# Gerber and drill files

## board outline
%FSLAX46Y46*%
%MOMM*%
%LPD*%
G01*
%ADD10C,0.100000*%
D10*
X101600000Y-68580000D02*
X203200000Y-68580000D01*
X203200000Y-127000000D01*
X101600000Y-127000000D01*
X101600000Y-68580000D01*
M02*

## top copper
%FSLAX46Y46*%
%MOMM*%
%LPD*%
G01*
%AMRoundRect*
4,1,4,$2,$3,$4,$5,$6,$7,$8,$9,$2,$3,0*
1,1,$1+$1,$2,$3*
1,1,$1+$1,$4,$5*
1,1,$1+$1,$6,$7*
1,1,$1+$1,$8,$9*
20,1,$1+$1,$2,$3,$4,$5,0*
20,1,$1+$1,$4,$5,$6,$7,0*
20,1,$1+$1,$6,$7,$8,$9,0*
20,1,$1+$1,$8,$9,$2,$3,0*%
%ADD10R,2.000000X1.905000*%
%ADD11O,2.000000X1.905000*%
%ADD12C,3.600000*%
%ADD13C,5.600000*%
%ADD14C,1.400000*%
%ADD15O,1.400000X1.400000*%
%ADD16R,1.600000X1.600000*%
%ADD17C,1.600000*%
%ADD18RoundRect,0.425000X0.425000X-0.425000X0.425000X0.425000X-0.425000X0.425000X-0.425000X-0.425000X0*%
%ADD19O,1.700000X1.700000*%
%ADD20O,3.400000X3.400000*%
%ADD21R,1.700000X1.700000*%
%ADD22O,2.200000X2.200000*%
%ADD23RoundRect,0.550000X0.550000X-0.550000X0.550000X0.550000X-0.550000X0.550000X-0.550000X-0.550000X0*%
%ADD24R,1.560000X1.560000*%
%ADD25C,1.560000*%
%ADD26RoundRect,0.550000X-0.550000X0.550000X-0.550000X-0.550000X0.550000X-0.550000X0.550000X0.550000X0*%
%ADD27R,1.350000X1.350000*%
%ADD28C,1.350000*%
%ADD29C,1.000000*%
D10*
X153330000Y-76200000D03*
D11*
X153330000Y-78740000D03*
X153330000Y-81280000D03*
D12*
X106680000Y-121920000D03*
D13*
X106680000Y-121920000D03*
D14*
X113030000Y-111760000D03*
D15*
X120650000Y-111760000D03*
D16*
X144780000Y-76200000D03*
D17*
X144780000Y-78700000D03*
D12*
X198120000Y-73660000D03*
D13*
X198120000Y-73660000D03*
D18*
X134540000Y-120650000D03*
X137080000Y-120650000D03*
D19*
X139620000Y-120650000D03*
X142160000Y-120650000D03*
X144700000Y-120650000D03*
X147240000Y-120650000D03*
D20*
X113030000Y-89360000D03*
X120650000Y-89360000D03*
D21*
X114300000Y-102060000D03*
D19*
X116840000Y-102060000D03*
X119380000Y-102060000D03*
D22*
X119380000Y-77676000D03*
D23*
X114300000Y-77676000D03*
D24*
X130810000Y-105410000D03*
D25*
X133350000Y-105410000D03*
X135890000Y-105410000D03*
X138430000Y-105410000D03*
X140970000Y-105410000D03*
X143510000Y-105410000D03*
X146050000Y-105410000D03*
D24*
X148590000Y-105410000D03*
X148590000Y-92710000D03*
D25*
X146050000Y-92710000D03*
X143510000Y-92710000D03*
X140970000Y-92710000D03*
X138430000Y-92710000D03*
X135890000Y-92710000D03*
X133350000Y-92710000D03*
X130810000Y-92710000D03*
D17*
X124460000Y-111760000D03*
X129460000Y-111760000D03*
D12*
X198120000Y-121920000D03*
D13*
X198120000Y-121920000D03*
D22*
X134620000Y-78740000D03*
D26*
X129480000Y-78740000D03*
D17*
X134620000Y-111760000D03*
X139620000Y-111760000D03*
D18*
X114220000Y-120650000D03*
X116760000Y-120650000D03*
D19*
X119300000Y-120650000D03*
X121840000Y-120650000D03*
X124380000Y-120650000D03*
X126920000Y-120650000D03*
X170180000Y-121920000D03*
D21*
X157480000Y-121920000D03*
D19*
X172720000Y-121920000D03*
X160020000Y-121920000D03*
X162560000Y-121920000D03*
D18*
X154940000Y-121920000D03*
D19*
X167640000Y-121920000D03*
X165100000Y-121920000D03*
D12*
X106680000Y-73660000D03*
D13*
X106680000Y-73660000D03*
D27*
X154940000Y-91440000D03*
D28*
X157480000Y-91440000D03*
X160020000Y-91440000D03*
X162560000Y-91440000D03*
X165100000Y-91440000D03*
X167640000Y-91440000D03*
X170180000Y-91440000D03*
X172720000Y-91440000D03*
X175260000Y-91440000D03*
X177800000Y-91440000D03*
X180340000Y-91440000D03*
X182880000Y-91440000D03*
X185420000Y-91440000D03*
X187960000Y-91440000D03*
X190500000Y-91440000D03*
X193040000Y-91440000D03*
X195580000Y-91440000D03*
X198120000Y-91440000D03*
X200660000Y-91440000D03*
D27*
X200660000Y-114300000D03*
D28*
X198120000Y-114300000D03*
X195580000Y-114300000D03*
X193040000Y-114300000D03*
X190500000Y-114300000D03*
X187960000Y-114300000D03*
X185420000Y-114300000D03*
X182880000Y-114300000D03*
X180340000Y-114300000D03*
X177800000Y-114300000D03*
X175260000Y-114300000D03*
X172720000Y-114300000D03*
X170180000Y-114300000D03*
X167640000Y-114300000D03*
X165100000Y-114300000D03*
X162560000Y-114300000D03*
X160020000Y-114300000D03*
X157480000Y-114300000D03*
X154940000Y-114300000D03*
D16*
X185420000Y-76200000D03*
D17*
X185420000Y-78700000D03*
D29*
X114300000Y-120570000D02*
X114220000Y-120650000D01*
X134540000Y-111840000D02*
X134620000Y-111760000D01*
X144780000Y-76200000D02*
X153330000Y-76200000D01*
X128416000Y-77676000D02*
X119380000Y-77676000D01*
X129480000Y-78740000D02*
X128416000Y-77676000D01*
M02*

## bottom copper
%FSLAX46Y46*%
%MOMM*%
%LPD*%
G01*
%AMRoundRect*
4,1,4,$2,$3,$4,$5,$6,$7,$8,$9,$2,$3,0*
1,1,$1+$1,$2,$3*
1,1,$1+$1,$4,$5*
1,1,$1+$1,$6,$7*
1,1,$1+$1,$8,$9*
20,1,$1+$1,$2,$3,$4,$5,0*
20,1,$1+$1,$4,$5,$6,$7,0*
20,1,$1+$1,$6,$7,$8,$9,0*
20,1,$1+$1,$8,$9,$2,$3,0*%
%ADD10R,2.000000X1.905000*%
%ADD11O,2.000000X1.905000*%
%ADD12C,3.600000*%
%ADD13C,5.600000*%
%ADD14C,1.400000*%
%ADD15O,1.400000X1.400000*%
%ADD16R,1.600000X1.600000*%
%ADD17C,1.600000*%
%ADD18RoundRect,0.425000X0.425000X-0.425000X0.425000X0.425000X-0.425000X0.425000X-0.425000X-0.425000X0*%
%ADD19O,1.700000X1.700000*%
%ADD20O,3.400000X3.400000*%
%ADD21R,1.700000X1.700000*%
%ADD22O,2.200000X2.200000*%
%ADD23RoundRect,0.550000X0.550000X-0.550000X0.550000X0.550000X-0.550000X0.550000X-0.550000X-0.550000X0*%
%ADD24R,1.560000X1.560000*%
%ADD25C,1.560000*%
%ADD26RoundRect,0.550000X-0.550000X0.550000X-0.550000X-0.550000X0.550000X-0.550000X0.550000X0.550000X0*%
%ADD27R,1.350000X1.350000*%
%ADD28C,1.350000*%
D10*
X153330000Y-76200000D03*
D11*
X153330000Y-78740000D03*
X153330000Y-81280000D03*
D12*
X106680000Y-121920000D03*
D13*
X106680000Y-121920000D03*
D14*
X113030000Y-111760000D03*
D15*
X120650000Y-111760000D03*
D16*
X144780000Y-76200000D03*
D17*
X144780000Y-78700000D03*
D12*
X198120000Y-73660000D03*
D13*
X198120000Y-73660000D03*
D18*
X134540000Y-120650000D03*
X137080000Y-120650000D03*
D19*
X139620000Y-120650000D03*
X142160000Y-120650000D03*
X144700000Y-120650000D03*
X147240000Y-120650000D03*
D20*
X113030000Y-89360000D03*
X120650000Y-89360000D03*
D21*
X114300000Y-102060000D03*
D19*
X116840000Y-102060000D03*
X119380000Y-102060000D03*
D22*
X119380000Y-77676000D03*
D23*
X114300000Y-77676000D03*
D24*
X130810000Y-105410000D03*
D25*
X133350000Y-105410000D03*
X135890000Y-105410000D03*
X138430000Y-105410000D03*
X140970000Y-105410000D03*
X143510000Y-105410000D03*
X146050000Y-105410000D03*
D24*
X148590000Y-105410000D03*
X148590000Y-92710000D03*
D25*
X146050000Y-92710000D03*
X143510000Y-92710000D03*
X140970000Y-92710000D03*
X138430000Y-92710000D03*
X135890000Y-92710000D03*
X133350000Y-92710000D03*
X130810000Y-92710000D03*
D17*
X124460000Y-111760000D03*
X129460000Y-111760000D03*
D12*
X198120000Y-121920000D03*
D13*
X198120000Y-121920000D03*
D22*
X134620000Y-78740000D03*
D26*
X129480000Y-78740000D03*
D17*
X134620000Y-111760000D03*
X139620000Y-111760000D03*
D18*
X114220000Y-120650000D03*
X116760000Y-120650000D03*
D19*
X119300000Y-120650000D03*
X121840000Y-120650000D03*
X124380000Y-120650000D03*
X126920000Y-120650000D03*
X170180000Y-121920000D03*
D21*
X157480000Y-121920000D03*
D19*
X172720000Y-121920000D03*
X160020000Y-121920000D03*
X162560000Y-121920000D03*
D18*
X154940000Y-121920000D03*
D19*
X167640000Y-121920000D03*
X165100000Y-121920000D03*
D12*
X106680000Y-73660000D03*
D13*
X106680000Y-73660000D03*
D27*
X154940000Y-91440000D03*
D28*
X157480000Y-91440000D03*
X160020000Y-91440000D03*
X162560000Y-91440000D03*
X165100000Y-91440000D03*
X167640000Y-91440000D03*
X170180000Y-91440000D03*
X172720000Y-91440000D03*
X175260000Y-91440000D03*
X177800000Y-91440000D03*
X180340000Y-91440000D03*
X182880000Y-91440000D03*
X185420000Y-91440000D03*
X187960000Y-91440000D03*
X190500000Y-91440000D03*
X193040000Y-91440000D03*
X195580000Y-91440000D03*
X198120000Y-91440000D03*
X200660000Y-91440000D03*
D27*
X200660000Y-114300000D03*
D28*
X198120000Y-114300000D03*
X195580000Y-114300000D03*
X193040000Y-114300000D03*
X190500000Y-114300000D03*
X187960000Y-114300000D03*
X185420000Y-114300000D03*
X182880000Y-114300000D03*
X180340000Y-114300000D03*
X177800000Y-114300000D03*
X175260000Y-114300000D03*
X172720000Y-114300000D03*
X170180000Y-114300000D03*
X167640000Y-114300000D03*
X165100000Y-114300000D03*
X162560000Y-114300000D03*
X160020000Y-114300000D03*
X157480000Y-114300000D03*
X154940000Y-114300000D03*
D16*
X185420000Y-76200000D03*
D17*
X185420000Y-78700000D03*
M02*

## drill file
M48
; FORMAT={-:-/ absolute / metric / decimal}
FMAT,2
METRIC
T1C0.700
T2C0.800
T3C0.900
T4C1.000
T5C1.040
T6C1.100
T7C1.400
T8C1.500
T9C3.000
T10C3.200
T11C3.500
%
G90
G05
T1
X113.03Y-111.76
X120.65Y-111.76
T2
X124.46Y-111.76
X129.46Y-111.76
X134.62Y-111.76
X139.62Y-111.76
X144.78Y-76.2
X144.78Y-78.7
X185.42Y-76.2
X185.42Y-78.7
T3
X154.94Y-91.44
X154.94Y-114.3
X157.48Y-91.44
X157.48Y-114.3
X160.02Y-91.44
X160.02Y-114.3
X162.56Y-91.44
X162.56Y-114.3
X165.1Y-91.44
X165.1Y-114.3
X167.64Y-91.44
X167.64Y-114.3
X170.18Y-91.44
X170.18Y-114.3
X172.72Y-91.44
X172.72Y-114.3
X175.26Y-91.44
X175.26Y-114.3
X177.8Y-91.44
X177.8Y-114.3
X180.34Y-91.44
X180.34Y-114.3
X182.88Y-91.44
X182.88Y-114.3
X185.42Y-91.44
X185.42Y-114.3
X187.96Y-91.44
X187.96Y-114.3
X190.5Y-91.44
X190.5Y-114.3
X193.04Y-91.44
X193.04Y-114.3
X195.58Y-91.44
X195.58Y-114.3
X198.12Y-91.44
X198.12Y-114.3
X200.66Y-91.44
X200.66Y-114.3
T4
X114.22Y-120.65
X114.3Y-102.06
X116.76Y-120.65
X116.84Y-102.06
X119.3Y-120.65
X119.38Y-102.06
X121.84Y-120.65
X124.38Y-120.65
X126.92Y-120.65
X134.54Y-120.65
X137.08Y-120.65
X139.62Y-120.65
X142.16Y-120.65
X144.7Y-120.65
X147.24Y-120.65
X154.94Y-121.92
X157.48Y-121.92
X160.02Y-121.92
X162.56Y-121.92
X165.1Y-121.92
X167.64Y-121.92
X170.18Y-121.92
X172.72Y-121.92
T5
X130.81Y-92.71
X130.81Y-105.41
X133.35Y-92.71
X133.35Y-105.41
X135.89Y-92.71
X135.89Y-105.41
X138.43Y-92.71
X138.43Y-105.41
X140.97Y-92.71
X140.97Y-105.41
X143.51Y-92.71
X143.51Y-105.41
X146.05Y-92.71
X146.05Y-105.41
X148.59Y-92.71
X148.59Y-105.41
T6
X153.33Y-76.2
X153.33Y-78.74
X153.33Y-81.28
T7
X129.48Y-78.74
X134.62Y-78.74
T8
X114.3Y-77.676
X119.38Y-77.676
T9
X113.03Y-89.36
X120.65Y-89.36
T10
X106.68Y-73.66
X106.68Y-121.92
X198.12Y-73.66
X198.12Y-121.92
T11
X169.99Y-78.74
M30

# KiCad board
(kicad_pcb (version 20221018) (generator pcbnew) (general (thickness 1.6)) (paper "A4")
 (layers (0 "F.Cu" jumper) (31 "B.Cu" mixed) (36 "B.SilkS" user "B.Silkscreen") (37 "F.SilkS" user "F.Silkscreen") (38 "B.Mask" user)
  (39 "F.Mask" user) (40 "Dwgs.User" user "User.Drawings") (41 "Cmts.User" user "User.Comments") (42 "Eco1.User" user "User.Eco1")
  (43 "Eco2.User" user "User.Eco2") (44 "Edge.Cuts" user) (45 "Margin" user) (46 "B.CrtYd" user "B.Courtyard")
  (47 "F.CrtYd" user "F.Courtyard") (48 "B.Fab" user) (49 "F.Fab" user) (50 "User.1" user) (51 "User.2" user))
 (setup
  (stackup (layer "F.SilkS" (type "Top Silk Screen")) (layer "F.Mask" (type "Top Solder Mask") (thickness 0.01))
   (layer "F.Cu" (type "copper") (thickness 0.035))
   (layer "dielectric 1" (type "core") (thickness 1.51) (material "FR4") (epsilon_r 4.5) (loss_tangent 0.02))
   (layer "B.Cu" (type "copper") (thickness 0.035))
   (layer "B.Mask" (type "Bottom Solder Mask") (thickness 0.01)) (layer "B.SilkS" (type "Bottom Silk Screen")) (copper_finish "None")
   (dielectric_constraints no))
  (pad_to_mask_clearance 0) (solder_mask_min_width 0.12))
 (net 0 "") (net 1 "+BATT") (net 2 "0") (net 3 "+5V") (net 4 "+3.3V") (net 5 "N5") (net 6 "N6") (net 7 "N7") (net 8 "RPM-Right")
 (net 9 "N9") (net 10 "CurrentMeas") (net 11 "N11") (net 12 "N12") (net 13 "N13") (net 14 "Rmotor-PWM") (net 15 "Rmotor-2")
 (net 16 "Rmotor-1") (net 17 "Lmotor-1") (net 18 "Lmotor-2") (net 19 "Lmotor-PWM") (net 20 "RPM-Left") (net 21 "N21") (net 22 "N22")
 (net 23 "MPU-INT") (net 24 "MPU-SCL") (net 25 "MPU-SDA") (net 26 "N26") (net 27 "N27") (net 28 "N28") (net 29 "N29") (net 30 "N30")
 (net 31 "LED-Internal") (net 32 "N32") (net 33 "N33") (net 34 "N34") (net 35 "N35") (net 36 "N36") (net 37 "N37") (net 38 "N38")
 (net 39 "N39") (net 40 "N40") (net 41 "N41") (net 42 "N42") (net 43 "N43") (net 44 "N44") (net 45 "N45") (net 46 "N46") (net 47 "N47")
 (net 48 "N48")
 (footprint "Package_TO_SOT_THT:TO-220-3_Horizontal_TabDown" (layer "F.Cu") (at 153.33 76.2 -90)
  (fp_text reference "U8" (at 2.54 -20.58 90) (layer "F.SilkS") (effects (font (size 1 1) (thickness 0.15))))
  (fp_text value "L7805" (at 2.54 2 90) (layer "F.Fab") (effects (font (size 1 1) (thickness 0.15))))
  (pad "" np_thru_hole oval (at 2.54 -16.66 270) (size 3.5 3.5) (drill 3.5) (layers "*.Cu" "*.Mask"))
  (pad "1" thru_hole rect (at 0 0 270) (size 1.905 2) (drill 1.1) (layers "*.Cu" "*.Mask") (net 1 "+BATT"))
  (pad "2" thru_hole oval (at 2.54 0 270) (size 1.905 2) (drill 1.1) (layers "*.Cu" "*.Mask") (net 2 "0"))
  (pad "3" thru_hole oval (at 5.08 0 270) (size 1.905 2) (drill 1.1) (layers "*.Cu" "*.Mask") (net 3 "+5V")))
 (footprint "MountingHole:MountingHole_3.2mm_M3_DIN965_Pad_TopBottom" (layer "F.Cu") (at 106.68 121.92)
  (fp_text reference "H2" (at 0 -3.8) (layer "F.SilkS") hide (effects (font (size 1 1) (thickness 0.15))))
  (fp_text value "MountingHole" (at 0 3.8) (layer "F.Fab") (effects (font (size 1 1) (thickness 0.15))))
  (pad "1" thru_hole circle (at 0 0) (size 3.6 3.6) (drill 3.2) (layers "*.Cu" "*.Mask"))
  (pad "1" connect circle (at 0 0) (size 5.6 5.6) (layers "F.Cu" "F.Mask"))
  (pad "1" connect circle (at 0 0) (size 5.6 5.6) (layers "B.Cu" "B.Mask")))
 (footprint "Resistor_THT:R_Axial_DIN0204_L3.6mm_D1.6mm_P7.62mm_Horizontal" (layer "F.Cu") (at 113.03 111.76)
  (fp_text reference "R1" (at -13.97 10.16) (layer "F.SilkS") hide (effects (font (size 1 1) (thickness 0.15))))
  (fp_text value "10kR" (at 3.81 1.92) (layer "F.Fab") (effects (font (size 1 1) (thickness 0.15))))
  (pad "1" thru_hole circle (at 0 0) (size 1.4 1.4) (drill 0.7) (layers "*.Cu" "*.Mask") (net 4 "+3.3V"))
  (pad "2" thru_hole oval (at 7.62 0) (size 1.4 1.4) (drill 0.7) (layers "*.Cu" "*.Mask") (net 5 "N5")))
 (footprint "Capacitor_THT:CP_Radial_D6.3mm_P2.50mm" (layer "F.Cu") (at 144.78 76.2 -90)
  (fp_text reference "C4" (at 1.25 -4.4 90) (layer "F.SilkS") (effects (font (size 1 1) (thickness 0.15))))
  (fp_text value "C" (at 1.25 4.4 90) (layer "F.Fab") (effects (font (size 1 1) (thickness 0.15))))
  (pad "1" thru_hole rect (at 0 0 270) (size 1.6 1.6) (drill 0.8) (layers "*.Cu" "*.Mask") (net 1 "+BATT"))
  (pad "2" thru_hole circle (at 2.5 0 270) (size 1.6 1.6) (drill 0.8) (layers "*.Cu" "*.Mask") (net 2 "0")))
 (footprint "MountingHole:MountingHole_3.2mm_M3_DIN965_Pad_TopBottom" (layer "F.Cu") (at 198.12 73.66)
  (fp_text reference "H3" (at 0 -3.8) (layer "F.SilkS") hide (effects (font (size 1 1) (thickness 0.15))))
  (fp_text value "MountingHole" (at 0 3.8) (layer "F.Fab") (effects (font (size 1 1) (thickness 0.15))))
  (pad "1" thru_hole circle (at 0 0) (size 3.6 3.6) (drill 3.2) (layers "*.Cu" "*.Mask"))
  (pad "1" connect circle (at 0 0) (size 5.6 5.6) (layers "F.Cu" "F.Mask"))
  (pad "1" connect circle (at 0 0) (size 5.6 5.6) (layers "B.Cu" "B.Mask")))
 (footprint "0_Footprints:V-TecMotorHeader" (layer "F.Cu") (at 141.2075 119.38 90)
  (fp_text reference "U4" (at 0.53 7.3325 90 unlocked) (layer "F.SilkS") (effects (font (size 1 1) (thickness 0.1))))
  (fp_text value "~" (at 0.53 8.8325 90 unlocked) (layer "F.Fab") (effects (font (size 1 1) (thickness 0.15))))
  (pad "1" thru_hole roundrect (at -1.27 -6.6675 90) (size 1.7 1.7) (drill 1) (layers "*.Cu" "*.Mask") (roundrect_rratio 0.25) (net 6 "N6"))
  (pad "2" thru_hole roundrect (at -1.27 -4.1275 90) (size 1.7 1.7) (drill 1) (layers "*.Cu" "*.Mask") (roundrect_rratio 0.25) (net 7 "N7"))
  (pad "3" thru_hole oval (at -1.27 -1.5875 90) (size 1.7 1.7) (drill 1) (layers "*.Cu" "*.Mask") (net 4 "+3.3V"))
  (pad "4" thru_hole oval (at -1.27 0.9525 90) (size 1.7 1.7) (drill 1) (layers "*.Cu" "*.Mask") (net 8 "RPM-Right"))
  (pad "5" thru_hole oval (at -1.27 3.4925 90) (size 1.7 1.7) (drill 1) (layers "*.Cu" "*.Mask") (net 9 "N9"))
  (pad "6" thru_hole oval (at -1.27 6.0325 90) (size 1.7 1.7) (drill 1) (layers "*.Cu" "*.Mask") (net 2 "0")))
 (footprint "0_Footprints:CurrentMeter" (layer "F.Cu") (at 116.84 102.06)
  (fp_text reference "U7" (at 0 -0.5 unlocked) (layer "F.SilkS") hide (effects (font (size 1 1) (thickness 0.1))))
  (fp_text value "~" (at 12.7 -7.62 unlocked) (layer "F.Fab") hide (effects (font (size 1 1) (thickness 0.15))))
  (pad "" thru_hole oval (at -3.81 -12.7 90) (size 3.4 3.4) (drill 3) (layers "*.Cu" "*.Mask"))
  (pad "" thru_hole oval (at 3.81 -12.7 90) (size 3.4 3.4) (drill 3) (layers "*.Cu" "*.Mask"))
  (pad "1" thru_hole rect (at -2.54 0 90) (size 1.7 1.7) (drill 1) (layers "*.Cu" "*.Mask") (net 2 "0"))
  (pad "2" thru_hole oval (at 0 0 90) (size 1.7 1.7) (drill 1) (layers "*.Cu" "*.Mask") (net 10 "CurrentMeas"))
  (pad "3" thru_hole oval (at 2.54 0 90) (size 1.7 1.7) (drill 1) (layers "*.Cu" "*.Mask") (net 3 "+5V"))
  (pad "p1" thru_hole oval (at 2.54 -24.384 90) (size 2.2 2.2) (drill 1.5) (layers "*.Cu" "*.Mask") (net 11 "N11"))
  (pad "p2" thru_hole roundrect (at -2.54 -24.384 90) (size 2.2 2.2) (drill 1.5) (layers "*.Cu" "*.Mask") (roundrect_rratio 0.25)
   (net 1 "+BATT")))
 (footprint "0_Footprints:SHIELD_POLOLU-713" (layer "F.Cu") (at 139.7 99.06 90)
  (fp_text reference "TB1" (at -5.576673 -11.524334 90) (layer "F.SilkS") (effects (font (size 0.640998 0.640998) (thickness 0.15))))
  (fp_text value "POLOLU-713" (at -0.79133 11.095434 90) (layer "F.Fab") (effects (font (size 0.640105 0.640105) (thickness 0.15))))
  (pad "1" thru_hole rect (at -6.35 -8.89 90) (size 1.56 1.56) (drill 1.04) (layers "*.Cu" "*.Mask") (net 2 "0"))
  (pad "2" thru_hole circle (at -6.35 -6.35 90) (size 1.56 1.56) (drill 1.04) (layers "*.Cu" "*.Mask") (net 4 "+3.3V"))
  (pad "3" thru_hole circle (at -6.35 -3.81 90) (size 1.56 1.56) (drill 1.04) (layers "*.Cu" "*.Mask") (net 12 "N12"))
  (pad "4" thru_hole circle (at -6.35 -1.27 90) (size 1.56 1.56) (drill 1.04) (layers "*.Cu" "*.Mask") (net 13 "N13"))
  (pad "5" thru_hole circle (at -6.35 1.27 90) (size 1.56 1.56) (drill 1.04) (layers "*.Cu" "*.Mask") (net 6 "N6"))
  (pad "6" thru_hole circle (at -6.35 3.81 90) (size 1.56 1.56) (drill 1.04) (layers "*.Cu" "*.Mask") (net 7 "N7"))
  (pad "7" thru_hole circle (at -6.35 6.35 90) (size 1.56 1.56) (drill 1.04) (layers "*.Cu" "*.Mask") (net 1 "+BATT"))
  (pad "8" thru_hole rect (at -6.35 8.89 90) (size 1.56 1.56) (drill 1.04) (layers "*.Cu" "*.Mask") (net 2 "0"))
  (pad "9" thru_hole rect (at 6.35 8.89 90) (size 1.56 1.56) (drill 1.04) (layers "*.Cu" "*.Mask") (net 2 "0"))
  (pad "10" thru_hole circle (at 6.35 6.35 90) (size 1.56 1.56) (drill 1.04) (layers "*.Cu" "*.Mask") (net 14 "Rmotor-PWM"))
  (pad "11" thru_hole circle (at 6.35 3.81 90) (size 1.56 1.56) (drill 1.04) (layers "*.Cu" "*.Mask") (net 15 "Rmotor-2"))
  (pad "12" thru_hole circle (at 6.35 1.27 90) (size 1.56 1.56) (drill 1.04) (layers "*.Cu" "*.Mask") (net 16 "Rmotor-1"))
  (pad "13" thru_hole circle (at 6.35 -1.27 90) (size 1.56 1.56) (drill 1.04) (layers "*.Cu" "*.Mask") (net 5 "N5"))
  (pad "14" thru_hole circle (at 6.35 -3.81 90) (size 1.56 1.56) (drill 1.04) (layers "*.Cu" "*.Mask") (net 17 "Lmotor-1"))
  (pad "15" thru_hole circle (at 6.35 -6.35 90) (size 1.56 1.56) (drill 1.04) (layers "*.Cu" "*.Mask") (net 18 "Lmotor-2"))
  (pad "16" thru_hole circle (at 6.35 -8.89 90) (size 1.56 1.56) (drill 1.04) (layers "*.Cu" "*.Mask") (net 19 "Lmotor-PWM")))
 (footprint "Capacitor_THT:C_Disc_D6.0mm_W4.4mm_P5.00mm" (layer "F.Cu") (at 124.46 111.76)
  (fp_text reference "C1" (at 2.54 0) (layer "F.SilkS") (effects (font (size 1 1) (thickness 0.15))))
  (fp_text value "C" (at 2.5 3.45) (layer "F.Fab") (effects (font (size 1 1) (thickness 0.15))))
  (pad "1" thru_hole circle (at 0 0) (size 1.6 1.6) (drill 0.8) (layers "*.Cu" "*.Mask") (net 12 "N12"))
  (pad "2" thru_hole circle (at 5 0) (size 1.6 1.6) (drill 0.8) (layers "*.Cu" "*.Mask") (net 13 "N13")))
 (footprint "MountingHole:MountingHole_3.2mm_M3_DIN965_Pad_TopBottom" (layer "F.Cu") (at 198.12 121.92)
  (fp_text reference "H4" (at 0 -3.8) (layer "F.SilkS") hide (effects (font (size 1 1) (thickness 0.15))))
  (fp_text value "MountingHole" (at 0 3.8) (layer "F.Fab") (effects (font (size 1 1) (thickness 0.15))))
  (pad "1" thru_hole circle (at 0 0) (size 3.6 3.6) (drill 3.2) (layers "*.Cu" "*.Mask"))
  (pad "1" connect circle (at 0 0) (size 5.6 5.6) (layers "F.Cu" "F.Mask"))
  (pad "1" connect circle (at 0 0) (size 5.6 5.6) (layers "B.Cu" "B.Mask")))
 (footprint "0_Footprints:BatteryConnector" (layer "F.Cu") (at 130.115 78.74 -90)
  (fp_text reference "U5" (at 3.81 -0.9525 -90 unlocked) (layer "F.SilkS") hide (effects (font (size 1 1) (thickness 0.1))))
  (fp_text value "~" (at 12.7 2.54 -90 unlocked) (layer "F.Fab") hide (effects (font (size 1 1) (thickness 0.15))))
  (pad "GND" thru_hole oval (at 0 -4.505 270) (size 2.2 2.2) (drill 1.4) (layers "*.Cu" "*.Mask") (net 2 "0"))
  (pad "Vbatt" thru_hole roundrect (at 0 0.635 270) (size 2.2 2.2) (drill 1.4) (layers "*.Cu" "*.Mask") (roundrect_rratio 0.25)
   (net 11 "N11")))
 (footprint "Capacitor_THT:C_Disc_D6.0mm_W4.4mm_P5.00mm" (layer "F.Cu") (at 134.62 111.76)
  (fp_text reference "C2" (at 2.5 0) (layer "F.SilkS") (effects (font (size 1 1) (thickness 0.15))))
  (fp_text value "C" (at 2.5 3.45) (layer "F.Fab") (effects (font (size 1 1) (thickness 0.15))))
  (pad "1" thru_hole circle (at 0 0) (size 1.6 1.6) (drill 0.8) (layers "*.Cu" "*.Mask") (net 6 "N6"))
  (pad "2" thru_hole circle (at 5 0) (size 1.6 1.6) (drill 0.8) (layers "*.Cu" "*.Mask") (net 7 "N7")))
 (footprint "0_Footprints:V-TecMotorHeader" (layer "F.Cu") (at 120.8875 119.38 90)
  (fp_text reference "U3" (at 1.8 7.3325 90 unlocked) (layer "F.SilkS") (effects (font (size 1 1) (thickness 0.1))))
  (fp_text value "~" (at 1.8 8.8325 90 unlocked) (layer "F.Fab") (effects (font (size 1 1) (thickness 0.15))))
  (pad "1" thru_hole roundrect (at -1.27 -6.6675 90) (size 1.7 1.7) (drill 1) (layers "*.Cu" "*.Mask") (roundrect_rratio 0.25)
   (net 12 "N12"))
  (pad "2" thru_hole roundrect (at -1.27 -4.1275 90) (size 1.7 1.7) (drill 1) (layers "*.Cu" "*.Mask") (roundrect_rratio 0.25)
   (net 13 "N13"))
  (pad "3" thru_hole oval (at -1.27 -1.5875 90) (size 1.7 1.7) (drill 1) (layers "*.Cu" "*.Mask") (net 4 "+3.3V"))
  (pad "4" thru_hole oval (at -1.27 0.9525 90) (size 1.7 1.7) (drill 1) (layers "*.Cu" "*.Mask") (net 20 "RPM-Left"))
  (pad "5" thru_hole oval (at -1.27 3.4925 90) (size 1.7 1.7) (drill 1) (layers "*.Cu" "*.Mask") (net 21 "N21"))
  (pad "6" thru_hole oval (at -1.27 6.0325 90) (size 1.7 1.7) (drill 1) (layers "*.Cu" "*.Mask") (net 2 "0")))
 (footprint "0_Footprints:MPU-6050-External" (layer "F.Cu") (at 172.72 121.92 -90)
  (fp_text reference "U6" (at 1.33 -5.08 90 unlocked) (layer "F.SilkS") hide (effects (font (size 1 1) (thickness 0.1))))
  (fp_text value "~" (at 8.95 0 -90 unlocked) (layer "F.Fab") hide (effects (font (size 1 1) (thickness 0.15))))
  (pad "ADO" thru_hole oval (at 0 2.54 90) (size 1.7 1.7) (drill 1) (layers "*.Cu" "*.Mask") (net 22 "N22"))
  (pad "GND" thru_hole rect (at 0 15.24 90) (size 1.7 1.7) (drill 1) (layers "*.Cu" "*.Mask") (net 2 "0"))
  (pad "INT" thru_hole oval (at 0 0 90) (size 1.7 1.7) (drill 1) (layers "*.Cu" "*.Mask") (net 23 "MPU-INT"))
  (pad "SCL" thru_hole oval (at 0 12.7 90) (size 1.7 1.7) (drill 1) (layers "*.Cu" "*.Mask") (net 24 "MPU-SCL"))
  (pad "SDA" thru_hole oval (at 0 10.16 90) (size 1.7 1.7) (drill 1) (layers "*.Cu" "*.Mask") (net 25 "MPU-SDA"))
  (pad "VCC" thru_hole roundrect (at 0 17.78 90) (size 1.7 1.7) (drill 1) (layers "*.Cu" "*.Mask") (roundrect_rratio 0.25) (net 4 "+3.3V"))
  (pad "XCL" thru_hole oval (at 0 5.08 90) (size 1.7 1.7) (drill 1) (layers "*.Cu" "*.Mask") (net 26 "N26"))
  (pad "XDA" thru_hole oval (at 0 7.62 90) (size 1.7 1.7) (drill 1) (layers "*.Cu" "*.Mask") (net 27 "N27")))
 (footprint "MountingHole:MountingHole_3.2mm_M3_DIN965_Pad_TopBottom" (layer "F.Cu") (at 106.68 73.66)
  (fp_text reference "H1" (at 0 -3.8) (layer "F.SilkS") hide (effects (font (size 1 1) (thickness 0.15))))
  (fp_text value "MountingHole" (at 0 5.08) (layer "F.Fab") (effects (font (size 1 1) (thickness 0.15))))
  (pad "1" thru_hole circle (at 0 0) (size 3.6 3.6) (drill 3.2) (layers "*.Cu" "*.Mask"))
  (pad "1" connect circle (at 0 0) (size 5.6 5.6) (layers "F.Cu" "F.Mask"))
  (pad "1" connect circle (at 0 0) (size 5.6 5.6) (layers "B.Cu" "B.Mask")))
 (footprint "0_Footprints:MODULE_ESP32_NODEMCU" (layer "F.Cu") (at 177.8 102.87 90)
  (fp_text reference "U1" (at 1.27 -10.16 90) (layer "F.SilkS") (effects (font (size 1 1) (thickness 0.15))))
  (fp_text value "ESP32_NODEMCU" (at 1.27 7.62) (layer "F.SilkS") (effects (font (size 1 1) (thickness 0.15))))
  (pad "J4_1" thru_hole rect (at 11.43 -22.86 90) (size 1.35 1.35) (drill 0.9) (layers "*.Cu" "*.Mask") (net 2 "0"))
  (pad "J4_2" thru_hole circle (at 11.43 -20.32 90) (size 1.35 1.35) (drill 0.9) (layers "*.Cu" "*.Mask") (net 23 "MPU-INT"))
  (pad "J4_3" thru_hole circle (at 11.43 -17.78 90) (size 1.35 1.35) (drill 0.9) (layers "*.Cu" "*.Mask") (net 24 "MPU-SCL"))
  (pad "J4_4" thru_hole circle (at 11.43 -15.24 90) (size 1.35 1.35) (drill 0.9) (layers "*.Cu" "*.Mask") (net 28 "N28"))
  (pad "J4_5" thru_hole circle (at 11.43 -12.7 90) (size 1.35 1.35) (drill 0.9) (layers "*.Cu" "*.Mask") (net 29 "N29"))
  (pad "J4_6" thru_hole circle (at 11.43 -10.16 90) (size 1.35 1.35) (drill 0.9) (layers "*.Cu" "*.Mask") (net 25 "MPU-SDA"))
  (pad "J4_7" thru_hole circle (at 11.43 -7.62 90) (size 1.35 1.35) (drill 0.9) (layers "*.Cu" "*.Mask") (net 2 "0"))
  (pad "J4_8" thru_hole circle (at 11.43 -5.08 90) (size 1.35 1.35) (drill 0.9) (layers "*.Cu" "*.Mask") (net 17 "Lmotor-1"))
  (pad "J4_9" thru_hole circle (at 11.43 -2.54 90) (size 1.35 1.35) (drill 0.9) (layers "*.Cu" "*.Mask") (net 18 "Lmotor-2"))
  (pad "J4_10" thru_hole circle (at 11.43 0 90) (size 1.35 1.35) (drill 0.9) (layers "*.Cu" "*.Mask") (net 19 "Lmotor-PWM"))
  (pad "J4_11" thru_hole circle (at 11.43 2.54 90) (size 1.35 1.35) (drill 0.9) (layers "*.Cu" "*.Mask") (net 16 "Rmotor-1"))
  (pad "J4_12" thru_hole circle (at 11.43 5.08 90) (size 1.35 1.35) (drill 0.9) (layers "*.Cu" "*.Mask") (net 15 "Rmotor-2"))
  (pad "J4_13" thru_hole circle (at 11.43 7.62 90) (size 1.35 1.35) (drill 0.9) (layers "*.Cu" "*.Mask") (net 14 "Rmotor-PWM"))
  (pad "J4_14" thru_hole circle (at 11.43 10.16 90) (size 1.35 1.35) (drill 0.9) (layers "*.Cu" "*.Mask") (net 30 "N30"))
  (pad "J4_15" thru_hole circle (at 11.43 12.7 90) (size 1.35 1.35) (drill 0.9) (layers "*.Cu" "*.Mask") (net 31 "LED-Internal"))
  (pad "J4_16" thru_hole circle (at 11.43 15.24 90) (size 1.35 1.35) (drill 0.9) (layers "*.Cu" "*.Mask") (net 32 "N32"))
  (pad "J4_17" thru_hole circle (at 11.43 17.78 90) (size 1.35 1.35) (drill 0.9) (layers "*.Cu" "*.Mask") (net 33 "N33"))
  (pad "J4_18" thru_hole circle (at 11.43 20.32 90) (size 1.35 1.35) (drill 0.9) (layers "*.Cu" "*.Mask") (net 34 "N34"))
  (pad "J4_19" thru_hole circle (at 11.43 22.86 90) (size 1.35 1.35) (drill 0.9) (layers "*.Cu" "*.Mask") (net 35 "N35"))
  (pad "J5_1" thru_hole rect (at -11.43 22.86 90) (size 1.35 1.35) (drill 0.9) (layers "*.Cu" "*.Mask") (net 3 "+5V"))
  (pad "J5_2" thru_hole circle (at -11.43 20.32 90) (size 1.35 1.35) (drill 0.9) (layers "*.Cu" "*.Mask") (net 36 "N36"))
  (pad "J5_3" thru_hole circle (at -11.43 17.78 90) (size 1.35 1.35) (drill 0.9) (layers "*.Cu" "*.Mask") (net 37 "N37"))
  (pad "J5_4" thru_hole circle (at -11.43 15.24 90) (size 1.35 1.35) (drill 0.9) (layers "*.Cu" "*.Mask") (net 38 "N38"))
  (pad "J5_5" thru_hole circle (at -11.43 12.7 90) (size 1.35 1.35) (drill 0.9) (layers "*.Cu" "*.Mask") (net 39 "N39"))
  (pad "J5_6" thru_hole circle (at -11.43 10.16 90) (size 1.35 1.35) (drill 0.9) (layers "*.Cu" "*.Mask") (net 2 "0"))
  (pad "J5_7" thru_hole circle (at -11.43 7.62 90) (size 1.35 1.35) (drill 0.9) (layers "*.Cu" "*.Mask") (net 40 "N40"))
  (pad "J5_8" thru_hole circle (at -11.43 5.08 90) (size 1.35 1.35) (drill 0.9) (layers "*.Cu" "*.Mask") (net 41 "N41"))
  (pad "J5_9" thru_hole circle (at -11.43 2.54 90) (size 1.35 1.35) (drill 0.9) (layers "*.Cu" "*.Mask") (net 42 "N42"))
  (pad "J5_10" thru_hole circle (at -11.43 0 90) (size 1.35 1.35) (drill 0.9) (layers "*.Cu" "*.Mask") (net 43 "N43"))
  (pad "J5_11" thru_hole circle (at -11.43 -2.54 90) (size 1.35 1.35) (drill 0.9) (layers "*.Cu" "*.Mask") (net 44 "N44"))
  (pad "J5_12" thru_hole circle (at -11.43 -5.08 90) (size 1.35 1.35) (drill 0.9) (layers "*.Cu" "*.Mask") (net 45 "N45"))
  (pad "J5_13" thru_hole circle (at -11.43 -7.62 90) (size 1.35 1.35) (drill 0.9) (layers "*.Cu" "*.Mask") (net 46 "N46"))
  (pad "J5_14" thru_hole circle (at -11.43 -10.16 90) (size 1.35 1.35) (drill 0.9) (layers "*.Cu" "*.Mask") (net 10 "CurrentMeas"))
  (pad "J5_15" thru_hole circle (at -11.43 -12.7 90) (size 1.35 1.35) (drill 0.9) (layers "*.Cu" "*.Mask") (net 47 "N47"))
  (pad "J5_16" thru_hole circle (at -11.43 -15.24 90) (size 1.35 1.35) (drill 0.9) (layers "*.Cu" "*.Mask") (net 8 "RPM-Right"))
  (pad "J5_17" thru_hole circle (at -11.43 -17.78 90) (size 1.35 1.35) (drill 0.9) (layers "*.Cu" "*.Mask") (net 20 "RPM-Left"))
  (pad "J5_18" thru_hole circle (at -11.43 -20.32 90) (size 1.35 1.35) (drill 0.9) (layers "*.Cu" "*.Mask") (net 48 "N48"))
  (pad "J5_19" thru_hole circle (at -11.43 -22.86 90) (size 1.35 1.35) (drill 0.9) (layers "*.Cu" "*.Mask") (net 4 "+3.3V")))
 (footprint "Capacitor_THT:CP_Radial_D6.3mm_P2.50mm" (layer "F.Cu") (at 185.42 76.2 -90)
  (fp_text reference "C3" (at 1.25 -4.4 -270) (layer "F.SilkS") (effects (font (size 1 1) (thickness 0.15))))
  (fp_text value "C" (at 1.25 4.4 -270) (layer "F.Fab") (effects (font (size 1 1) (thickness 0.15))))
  (pad "1" thru_hole rect (at 0 0 270) (size 1.6 1.6) (drill 0.8) (layers "*.Cu" "*.Mask") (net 3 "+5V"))
  (pad "2" thru_hole circle (at 2.5 0 270) (size 1.6 1.6) (drill 0.8) (layers "*.Cu" "*.Mask") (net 2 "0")))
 (gr_rect (start 101.6 68.58) (end 203.2 127) (stroke (width 0.1) (type default)) (fill none) (layer "Edge.Cuts"))
 (segment (start 114.3 120.57) (end 114.22 120.65) (width 1) (layer "F.Cu") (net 12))
 (segment (start 134.54 111.84) (end 134.62 111.76) (width 1) (layer "F.Cu") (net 6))
 (segment (start 144.78 76.2) (end 153.33 76.2) (width 1) (layer "F.Cu") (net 1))
 (segment (start 128.416 77.676) (end 119.38 77.676) (width 1) (layer "F.Cu") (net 11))
 (segment (start 129.48 78.74) (end 128.416 77.676) (width 1) (layer "F.Cu") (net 11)))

